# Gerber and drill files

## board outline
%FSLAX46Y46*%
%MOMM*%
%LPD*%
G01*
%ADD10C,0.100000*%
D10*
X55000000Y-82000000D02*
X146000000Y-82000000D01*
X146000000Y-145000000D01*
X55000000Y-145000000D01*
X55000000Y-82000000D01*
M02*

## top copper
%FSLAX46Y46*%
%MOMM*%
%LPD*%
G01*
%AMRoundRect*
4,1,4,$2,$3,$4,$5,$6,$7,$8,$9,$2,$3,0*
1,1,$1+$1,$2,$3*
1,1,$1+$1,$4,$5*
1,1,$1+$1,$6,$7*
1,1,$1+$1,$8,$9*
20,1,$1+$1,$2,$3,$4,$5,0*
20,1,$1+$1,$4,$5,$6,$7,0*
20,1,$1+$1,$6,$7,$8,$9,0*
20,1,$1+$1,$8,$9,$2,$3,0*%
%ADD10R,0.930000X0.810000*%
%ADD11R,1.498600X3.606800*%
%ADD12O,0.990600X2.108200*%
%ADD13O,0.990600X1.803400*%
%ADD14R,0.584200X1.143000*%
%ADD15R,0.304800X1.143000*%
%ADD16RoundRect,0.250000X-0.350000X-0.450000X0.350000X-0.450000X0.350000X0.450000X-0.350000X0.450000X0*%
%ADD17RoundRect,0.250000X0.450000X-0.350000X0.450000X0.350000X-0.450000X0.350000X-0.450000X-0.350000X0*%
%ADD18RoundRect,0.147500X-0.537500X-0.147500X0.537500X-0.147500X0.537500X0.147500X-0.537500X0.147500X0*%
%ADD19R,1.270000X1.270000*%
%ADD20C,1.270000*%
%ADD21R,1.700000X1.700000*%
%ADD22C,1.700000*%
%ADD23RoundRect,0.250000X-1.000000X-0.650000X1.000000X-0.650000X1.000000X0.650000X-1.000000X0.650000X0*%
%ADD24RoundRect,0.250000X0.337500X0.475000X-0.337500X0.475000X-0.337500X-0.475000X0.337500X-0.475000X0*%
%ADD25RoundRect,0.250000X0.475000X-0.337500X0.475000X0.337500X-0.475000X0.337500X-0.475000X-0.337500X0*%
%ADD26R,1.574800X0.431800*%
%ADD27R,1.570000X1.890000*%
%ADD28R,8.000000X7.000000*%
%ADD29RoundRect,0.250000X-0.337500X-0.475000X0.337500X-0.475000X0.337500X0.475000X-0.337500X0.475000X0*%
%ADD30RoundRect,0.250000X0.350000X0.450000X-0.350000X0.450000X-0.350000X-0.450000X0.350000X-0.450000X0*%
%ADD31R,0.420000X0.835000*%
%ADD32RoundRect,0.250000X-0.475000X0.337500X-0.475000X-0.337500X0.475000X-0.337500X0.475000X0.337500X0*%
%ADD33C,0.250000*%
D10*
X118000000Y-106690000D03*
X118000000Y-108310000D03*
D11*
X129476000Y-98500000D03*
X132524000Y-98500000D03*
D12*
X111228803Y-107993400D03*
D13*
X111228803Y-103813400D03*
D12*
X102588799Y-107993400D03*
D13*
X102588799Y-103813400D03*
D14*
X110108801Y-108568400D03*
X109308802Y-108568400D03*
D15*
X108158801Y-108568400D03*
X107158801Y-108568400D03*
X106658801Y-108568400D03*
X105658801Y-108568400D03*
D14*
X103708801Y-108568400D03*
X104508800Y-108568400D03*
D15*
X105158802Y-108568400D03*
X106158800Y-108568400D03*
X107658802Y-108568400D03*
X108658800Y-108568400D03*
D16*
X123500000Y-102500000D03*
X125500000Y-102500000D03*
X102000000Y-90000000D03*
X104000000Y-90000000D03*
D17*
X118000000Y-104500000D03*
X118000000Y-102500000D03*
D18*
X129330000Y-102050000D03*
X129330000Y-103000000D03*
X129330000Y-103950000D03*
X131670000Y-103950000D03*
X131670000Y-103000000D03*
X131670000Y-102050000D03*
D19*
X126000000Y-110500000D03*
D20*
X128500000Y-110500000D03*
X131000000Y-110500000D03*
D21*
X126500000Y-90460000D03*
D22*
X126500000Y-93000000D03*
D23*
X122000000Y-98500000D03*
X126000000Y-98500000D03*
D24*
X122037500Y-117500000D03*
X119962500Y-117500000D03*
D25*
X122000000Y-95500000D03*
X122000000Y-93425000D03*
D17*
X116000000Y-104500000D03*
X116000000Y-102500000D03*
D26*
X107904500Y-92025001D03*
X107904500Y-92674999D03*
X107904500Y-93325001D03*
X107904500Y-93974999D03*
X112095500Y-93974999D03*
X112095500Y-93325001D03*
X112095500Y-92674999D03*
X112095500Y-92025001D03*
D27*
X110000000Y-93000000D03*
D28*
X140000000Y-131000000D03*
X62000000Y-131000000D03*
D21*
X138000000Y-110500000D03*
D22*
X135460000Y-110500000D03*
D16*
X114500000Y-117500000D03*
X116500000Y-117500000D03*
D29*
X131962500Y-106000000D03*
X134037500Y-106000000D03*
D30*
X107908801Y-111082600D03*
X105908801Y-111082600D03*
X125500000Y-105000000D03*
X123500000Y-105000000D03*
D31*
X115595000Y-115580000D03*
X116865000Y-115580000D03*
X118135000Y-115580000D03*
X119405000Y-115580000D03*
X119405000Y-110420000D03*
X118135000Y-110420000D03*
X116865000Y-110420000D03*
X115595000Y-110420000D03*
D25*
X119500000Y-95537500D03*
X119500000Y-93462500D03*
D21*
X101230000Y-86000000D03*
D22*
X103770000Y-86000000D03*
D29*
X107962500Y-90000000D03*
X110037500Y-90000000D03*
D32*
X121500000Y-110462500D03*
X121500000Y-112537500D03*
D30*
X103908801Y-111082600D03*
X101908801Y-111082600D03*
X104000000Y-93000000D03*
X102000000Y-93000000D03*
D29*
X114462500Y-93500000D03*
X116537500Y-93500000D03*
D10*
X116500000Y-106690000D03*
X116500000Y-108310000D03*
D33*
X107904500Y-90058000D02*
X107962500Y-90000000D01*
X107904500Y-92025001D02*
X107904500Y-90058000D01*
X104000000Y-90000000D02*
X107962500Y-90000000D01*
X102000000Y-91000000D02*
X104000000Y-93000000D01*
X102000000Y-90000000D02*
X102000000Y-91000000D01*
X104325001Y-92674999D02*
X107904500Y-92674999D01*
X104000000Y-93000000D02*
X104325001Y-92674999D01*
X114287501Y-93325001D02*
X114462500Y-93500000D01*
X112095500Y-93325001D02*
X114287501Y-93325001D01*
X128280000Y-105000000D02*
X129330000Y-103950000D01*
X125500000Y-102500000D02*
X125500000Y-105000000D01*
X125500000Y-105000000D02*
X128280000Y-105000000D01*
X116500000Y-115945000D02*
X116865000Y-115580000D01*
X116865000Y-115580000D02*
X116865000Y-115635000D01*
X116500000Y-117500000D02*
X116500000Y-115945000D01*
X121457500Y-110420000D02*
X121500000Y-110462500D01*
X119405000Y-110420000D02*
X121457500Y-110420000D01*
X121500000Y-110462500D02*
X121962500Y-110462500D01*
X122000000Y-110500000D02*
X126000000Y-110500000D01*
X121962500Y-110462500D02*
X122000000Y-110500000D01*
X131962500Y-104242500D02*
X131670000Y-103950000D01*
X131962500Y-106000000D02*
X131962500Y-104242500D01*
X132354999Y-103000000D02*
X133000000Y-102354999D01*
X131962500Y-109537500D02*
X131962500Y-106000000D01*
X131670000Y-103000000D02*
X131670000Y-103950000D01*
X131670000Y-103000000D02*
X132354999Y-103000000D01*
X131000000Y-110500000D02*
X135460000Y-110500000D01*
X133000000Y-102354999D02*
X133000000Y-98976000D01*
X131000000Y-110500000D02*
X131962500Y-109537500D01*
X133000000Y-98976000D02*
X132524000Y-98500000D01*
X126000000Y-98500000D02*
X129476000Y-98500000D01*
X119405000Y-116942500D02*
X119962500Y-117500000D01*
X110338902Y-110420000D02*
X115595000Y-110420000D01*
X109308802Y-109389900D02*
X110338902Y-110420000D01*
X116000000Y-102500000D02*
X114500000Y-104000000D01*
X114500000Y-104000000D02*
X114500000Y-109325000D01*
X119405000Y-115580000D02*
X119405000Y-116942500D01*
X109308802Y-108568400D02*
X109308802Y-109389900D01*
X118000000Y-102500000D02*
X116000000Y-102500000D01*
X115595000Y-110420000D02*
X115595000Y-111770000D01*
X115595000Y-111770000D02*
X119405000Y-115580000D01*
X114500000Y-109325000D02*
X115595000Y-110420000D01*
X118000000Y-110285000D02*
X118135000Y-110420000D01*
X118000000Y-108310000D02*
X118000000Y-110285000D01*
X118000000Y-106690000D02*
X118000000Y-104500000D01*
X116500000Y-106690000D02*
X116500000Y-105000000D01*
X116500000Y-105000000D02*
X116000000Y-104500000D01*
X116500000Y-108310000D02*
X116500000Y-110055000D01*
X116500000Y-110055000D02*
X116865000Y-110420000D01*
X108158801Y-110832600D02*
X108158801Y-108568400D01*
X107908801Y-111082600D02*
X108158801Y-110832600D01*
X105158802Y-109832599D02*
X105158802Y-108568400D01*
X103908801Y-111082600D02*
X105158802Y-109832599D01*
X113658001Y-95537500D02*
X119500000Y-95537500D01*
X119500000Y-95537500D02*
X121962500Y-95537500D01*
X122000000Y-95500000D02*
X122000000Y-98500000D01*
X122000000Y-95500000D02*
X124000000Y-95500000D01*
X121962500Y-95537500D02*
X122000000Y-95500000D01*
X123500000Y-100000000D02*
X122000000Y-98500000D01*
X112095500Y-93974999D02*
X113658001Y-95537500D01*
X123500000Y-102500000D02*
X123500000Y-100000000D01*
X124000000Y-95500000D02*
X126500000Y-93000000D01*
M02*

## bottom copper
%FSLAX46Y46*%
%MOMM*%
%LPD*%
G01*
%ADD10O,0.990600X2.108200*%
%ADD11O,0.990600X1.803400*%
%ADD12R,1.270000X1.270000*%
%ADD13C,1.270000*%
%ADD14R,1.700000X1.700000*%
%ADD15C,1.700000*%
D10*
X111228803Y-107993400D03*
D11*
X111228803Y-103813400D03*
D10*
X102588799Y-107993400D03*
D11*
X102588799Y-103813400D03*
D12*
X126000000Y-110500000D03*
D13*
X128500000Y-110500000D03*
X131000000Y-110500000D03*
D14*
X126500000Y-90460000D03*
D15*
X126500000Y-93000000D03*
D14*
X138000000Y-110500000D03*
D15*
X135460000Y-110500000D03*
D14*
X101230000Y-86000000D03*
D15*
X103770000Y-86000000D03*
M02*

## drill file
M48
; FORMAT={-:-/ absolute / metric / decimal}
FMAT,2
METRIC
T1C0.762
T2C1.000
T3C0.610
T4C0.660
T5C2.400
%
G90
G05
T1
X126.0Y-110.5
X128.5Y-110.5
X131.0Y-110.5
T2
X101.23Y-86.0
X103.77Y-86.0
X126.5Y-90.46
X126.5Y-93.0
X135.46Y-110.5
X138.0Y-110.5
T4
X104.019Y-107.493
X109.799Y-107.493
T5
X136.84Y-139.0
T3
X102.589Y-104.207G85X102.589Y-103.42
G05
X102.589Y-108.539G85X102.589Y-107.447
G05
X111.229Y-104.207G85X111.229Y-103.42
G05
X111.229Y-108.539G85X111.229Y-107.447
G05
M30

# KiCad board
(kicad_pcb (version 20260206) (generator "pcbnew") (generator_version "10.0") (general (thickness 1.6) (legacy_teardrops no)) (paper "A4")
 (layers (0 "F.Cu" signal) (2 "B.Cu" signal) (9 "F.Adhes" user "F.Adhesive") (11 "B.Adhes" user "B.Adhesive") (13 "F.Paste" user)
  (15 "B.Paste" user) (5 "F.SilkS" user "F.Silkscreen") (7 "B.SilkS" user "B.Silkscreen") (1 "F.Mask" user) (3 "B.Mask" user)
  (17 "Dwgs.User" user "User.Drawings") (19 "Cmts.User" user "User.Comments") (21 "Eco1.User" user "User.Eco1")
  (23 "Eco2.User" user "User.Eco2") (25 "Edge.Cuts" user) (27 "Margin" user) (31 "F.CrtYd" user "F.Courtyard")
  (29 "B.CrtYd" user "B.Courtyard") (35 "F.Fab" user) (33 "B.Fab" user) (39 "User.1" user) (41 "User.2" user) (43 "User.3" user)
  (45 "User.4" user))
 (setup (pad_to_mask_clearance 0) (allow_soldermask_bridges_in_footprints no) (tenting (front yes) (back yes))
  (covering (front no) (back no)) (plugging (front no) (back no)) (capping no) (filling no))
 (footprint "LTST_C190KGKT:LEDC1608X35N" (layer "F.Cu") (at 118 107.5 90)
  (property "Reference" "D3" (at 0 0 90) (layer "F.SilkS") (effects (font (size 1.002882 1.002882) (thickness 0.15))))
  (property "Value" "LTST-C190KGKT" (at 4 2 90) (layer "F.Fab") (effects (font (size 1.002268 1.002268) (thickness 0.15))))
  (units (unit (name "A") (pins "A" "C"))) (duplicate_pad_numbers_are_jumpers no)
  (pad "A" smd rect (at 0.81 0 90) (size 0.81 0.93) (layers "F.Cu" "F.Mask" "F.Paste") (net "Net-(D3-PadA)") (solder_mask_margin 0.102))
  (pad "C" smd rect (at -0.81 0 90) (size 0.81 0.93) (layers "F.Cu" "F.Mask" "F.Paste") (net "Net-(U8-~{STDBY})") (solder_mask_margin 0.102)))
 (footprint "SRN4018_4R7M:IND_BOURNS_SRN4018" (layer "F.Cu") (at 131 98.5)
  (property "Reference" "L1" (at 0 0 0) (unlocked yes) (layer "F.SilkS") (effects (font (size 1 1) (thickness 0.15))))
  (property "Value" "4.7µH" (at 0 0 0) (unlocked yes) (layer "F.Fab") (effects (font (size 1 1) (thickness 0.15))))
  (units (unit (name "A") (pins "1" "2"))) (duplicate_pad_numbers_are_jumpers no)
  (pad "1" smd rect (at -1.524 0) (size 1.4986 3.6068) (layers "F.Cu" "F.Mask" "F.Paste") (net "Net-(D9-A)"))
  (pad "2" smd rect (at 1.524 0) (size 1.4986 3.6068) (layers "F.Cu" "F.Mask" "F.Paste") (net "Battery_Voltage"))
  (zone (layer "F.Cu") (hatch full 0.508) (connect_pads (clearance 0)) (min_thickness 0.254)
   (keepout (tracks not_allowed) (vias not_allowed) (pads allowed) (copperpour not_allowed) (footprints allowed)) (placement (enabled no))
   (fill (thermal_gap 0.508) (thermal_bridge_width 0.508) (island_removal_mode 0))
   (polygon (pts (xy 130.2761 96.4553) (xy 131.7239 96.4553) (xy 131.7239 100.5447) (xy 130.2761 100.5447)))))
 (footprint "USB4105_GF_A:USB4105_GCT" (layer "F.Cu") (at 106.908801 105.0826 180)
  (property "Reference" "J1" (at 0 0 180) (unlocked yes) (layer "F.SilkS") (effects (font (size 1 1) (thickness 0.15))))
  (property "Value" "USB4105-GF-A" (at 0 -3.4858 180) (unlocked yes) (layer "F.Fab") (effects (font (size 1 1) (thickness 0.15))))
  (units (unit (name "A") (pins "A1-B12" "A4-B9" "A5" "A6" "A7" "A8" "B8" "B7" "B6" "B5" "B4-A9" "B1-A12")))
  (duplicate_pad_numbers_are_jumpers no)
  (pad "" np_thru_hole oval (at -4.320002 -2.9108 180) (size 0.9906 2.1082) (drill oval 0.6096 1.7018) (layers "*.Cu" "*.Mask"))
  (pad "" np_thru_hole oval (at -4.320002 1.2692 180) (size 0.9906 1.8034) (drill oval 0.6096 1.397) (layers "*.Cu" "*.Mask"))
  (pad "" np_thru_hole circle (at -2.889999 -2.410801 180) (size 0.6604 0.6604) (drill 0.6604) (layers "*.Cu" "*.Mask"))
  (pad "" np_thru_hole circle (at 2.889999 -2.410801 180) (size 0.6604 0.6604) (drill 0.6604) (layers "*.Cu" "*.Mask"))
  (pad "" np_thru_hole oval (at 4.320002 -2.9108 180) (size 0.9906 2.1082) (drill oval 0.6096 1.7018) (layers "*.Cu" "*.Mask"))
  (pad "" np_thru_hole oval (at 4.320002 1.2692 180) (size 0.9906 1.8034) (drill oval 0.6096 1.397) (layers "*.Cu" "*.Mask"))
  (pad "A1-B12" smd rect (at -3.2 -3.4858 180) (size 0.5842 1.143) (layers "F.Cu" "F.Mask" "F.Paste") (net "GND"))
  (pad "A4-B9" smd rect (at -2.400001 -3.4858 180) (size 0.5842 1.143) (layers "F.Cu" "F.Mask" "F.Paste") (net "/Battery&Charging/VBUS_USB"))
  (pad "A5" smd rect (at -1.25 -3.4858 180) (size 0.3048 1.143) (layers "F.Cu" "F.Mask" "F.Paste") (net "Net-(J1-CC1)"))
  (pad "A6" smd rect (at -0.25 -3.4858 180) (size 0.3048 1.143) (layers "F.Cu" "F.Mask" "F.Paste") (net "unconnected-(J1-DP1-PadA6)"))
  (pad "A7" smd rect (at 0.25 -3.4858 180) (size 0.3048 1.143) (layers "F.Cu" "F.Mask" "F.Paste") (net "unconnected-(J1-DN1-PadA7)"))
  (pad "A8" smd rect (at 1.25 -3.4858 180) (size 0.3048 1.143) (layers "F.Cu" "F.Mask" "F.Paste") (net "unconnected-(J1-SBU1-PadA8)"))
  (pad "B1-A12" smd rect (at 3.2 -3.4858 180) (size 0.5842 1.143) (layers "F.Cu" "F.Mask" "F.Paste") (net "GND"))
  (pad "B4-A9" smd rect (at 2.400001 -3.4858 180) (size 0.5842 1.143) (layers "F.Cu" "F.Mask" "F.Paste")
   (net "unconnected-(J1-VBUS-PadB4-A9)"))
  (pad "B5" smd rect (at 1.749999 -3.4858 180) (size 0.3048 1.143) (layers "F.Cu" "F.Mask" "F.Paste") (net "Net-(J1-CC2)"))
  (pad "B6" smd rect (at 0.750001 -3.4858 180) (size 0.3048 1.143) (layers "F.Cu" "F.Mask" "F.Paste") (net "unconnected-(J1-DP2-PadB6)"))
  (pad "B7" smd rect (at -0.750001 -3.4858 180) (size 0.3048 1.143) (layers "F.Cu" "F.Mask" "F.Paste") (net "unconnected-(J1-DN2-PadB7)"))
  (pad "B8" smd rect (at -1.749999 -3.4858 180) (size 0.3048 1.143) (layers "F.Cu" "F.Mask" "F.Paste") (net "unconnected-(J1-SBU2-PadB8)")))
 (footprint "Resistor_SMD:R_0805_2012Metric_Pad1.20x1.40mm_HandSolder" (layer "F.Cu") (at 124.5 102.5)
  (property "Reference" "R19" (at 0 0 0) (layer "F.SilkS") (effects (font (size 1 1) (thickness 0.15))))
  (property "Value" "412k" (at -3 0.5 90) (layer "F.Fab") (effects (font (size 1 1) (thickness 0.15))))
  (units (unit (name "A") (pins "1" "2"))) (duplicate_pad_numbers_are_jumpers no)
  (pad "1" smd roundrect (at -1 0) (size 1.2 1.4) (layers "F.Cu" "F.Mask" "F.Paste") (roundrect_rratio 0.208333)
   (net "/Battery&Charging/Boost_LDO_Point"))
  (pad "2" smd roundrect (at 1 0) (size 1.2 1.4) (layers "F.Cu" "F.Mask" "F.Paste") (roundrect_rratio 0.208333) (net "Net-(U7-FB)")))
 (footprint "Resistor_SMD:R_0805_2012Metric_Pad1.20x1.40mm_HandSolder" (layer "F.Cu") (at 103 90)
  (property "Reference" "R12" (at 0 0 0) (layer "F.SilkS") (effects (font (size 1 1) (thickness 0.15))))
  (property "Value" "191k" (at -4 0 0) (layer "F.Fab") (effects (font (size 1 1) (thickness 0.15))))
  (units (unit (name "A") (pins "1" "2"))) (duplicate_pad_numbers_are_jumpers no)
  (pad "1" smd roundrect (at -1 0) (size 1.2 1.4) (layers "F.Cu" "F.Mask" "F.Paste") (roundrect_rratio 0.208333) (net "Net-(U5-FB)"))
  (pad "2" smd roundrect (at 1 0) (size 1.2 1.4) (layers "F.Cu" "F.Mask" "F.Paste") (roundrect_rratio 0.208333) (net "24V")))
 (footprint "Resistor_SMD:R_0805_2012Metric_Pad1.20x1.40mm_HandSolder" (layer "F.Cu") (at 118 103.5 90)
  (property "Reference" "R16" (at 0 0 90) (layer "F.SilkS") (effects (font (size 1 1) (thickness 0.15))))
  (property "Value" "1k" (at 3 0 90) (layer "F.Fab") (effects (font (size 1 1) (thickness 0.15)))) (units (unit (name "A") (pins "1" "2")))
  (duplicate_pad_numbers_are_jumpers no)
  (pad "1" smd roundrect (at -1 0 90) (size 1.2 1.4) (layers "F.Cu" "F.Mask" "F.Paste") (roundrect_rratio 0.208333) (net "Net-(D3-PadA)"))
  (pad "2" smd roundrect (at 1 0 90) (size 1.2 1.4) (layers "F.Cu" "F.Mask" "F.Paste") (roundrect_rratio 0.208333)
   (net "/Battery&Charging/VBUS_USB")))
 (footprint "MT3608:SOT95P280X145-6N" (layer "F.Cu") (at 130.5 103)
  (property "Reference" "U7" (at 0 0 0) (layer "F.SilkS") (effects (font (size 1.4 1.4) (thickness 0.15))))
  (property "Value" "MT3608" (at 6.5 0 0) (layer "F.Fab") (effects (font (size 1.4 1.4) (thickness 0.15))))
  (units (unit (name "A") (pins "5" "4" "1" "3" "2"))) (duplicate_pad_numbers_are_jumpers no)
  (pad "1" smd roundrect (at -1.17 -0.95) (size 1.37 0.59) (layers "F.Cu" "F.Mask" "F.Paste") (roundrect_rratio 0.25) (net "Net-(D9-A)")
   (solder_mask_margin 0.102))
  (pad "2" smd roundrect (at -1.17 0) (size 1.37 0.59) (layers "F.Cu" "F.Mask" "F.Paste") (roundrect_rratio 0.25) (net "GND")
   (solder_mask_margin 0.102))
  (pad "3" smd roundrect (at -1.17 0.95) (size 1.37 0.59) (layers "F.Cu" "F.Mask" "F.Paste") (roundrect_rratio 0.25) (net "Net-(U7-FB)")
   (solder_mask_margin 0.102))
  (pad "4" smd roundrect (at 1.17 0.95) (size 1.37 0.59) (layers "F.Cu" "F.Mask" "F.Paste") (roundrect_rratio 0.25) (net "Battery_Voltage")
   (solder_mask_margin 0.102))
  (pad "5" smd roundrect (at 1.17 0) (size 1.37 0.59) (layers "F.Cu" "F.Mask" "F.Paste") (roundrect_rratio 0.25) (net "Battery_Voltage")
   (solder_mask_margin 0.102))
  (pad "6" smd roundrect (at 1.17 -0.95) (size 1.37 0.59) (layers "F.Cu" "F.Mask" "F.Paste") (roundrect_rratio 0.25)
   (solder_mask_margin 0.102)))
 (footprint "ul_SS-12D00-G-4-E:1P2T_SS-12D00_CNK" (layer "F.Cu") (at 126 110.5 90)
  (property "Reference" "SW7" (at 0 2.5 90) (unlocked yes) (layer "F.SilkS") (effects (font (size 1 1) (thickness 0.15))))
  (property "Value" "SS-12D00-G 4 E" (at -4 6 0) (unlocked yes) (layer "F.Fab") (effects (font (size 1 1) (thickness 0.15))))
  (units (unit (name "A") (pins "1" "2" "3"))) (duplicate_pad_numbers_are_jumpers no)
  (pad "1" thru_hole rect (at 0 0 90) (size 1.27 1.27) (drill 0.762) (layers "*.Cu" "*.Mask") (remove_unused_layers no) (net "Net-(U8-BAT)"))
  (pad "2" thru_hole circle (at 0 2.5 90) (size 1.27 1.27) (drill 0.762) (layers "*.Cu" "*.Mask") (remove_unused_layers no)
   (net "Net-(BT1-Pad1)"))
  (pad "3" thru_hole circle (at 0 5 90) (size 1.27 1.27) (drill 0.762) (layers "*.Cu" "*.Mask") (remove_unused_layers no)
   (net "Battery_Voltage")))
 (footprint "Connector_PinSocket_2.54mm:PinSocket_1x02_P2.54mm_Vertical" (layer "F.Cu") (at 126.5 90.46)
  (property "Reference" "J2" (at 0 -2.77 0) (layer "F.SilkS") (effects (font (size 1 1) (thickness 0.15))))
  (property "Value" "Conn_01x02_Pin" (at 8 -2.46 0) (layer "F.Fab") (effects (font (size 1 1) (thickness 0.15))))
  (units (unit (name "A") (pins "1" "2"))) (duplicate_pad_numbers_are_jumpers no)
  (pad "1" thru_hole rect (at 0 0) (size 1.7 1.7) (drill 1) (layers "*.Cu" "*.Mask") (remove_unused_layers no) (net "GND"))
  (pad "2" thru_hole circle (at 0 2.54) (size 1.7 1.7) (drill 1) (layers "*.Cu" "*.Mask") (remove_unused_layers no)
   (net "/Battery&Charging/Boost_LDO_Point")))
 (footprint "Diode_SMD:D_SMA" (layer "F.Cu") (at 124 98.5)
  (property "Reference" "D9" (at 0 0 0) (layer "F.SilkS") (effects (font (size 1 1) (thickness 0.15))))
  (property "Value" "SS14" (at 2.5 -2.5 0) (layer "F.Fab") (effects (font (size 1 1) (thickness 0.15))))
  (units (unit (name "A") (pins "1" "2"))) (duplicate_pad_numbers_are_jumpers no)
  (pad "1" smd roundrect (at -2 0) (size 2.5 1.8) (layers "F.Cu" "F.Mask" "F.Paste") (roundrect_rratio 0.1388888889)
   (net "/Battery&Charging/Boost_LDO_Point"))
  (pad "2" smd roundrect (at 2 0) (size 2.5 1.8) (layers "F.Cu" "F.Mask" "F.Paste") (roundrect_rratio 0.1388888889) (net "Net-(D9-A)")))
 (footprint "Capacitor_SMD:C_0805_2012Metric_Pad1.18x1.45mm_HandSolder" (layer "F.Cu") (at 121 117.5 180)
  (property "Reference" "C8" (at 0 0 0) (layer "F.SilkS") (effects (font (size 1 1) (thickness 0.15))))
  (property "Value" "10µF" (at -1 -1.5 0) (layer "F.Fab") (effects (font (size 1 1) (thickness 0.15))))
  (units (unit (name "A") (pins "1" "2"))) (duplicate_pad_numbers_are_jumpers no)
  (pad "1" smd roundrect (at -1.0375 0 180) (size 1.175 1.45) (layers "F.Cu" "F.Mask" "F.Paste") (roundrect_rratio 0.212766) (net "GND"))
  (pad "2" smd roundrect (at 1.0375 0 180) (size 1.175 1.45) (layers "F.Cu" "F.Mask" "F.Paste") (roundrect_rratio 0.212766)
   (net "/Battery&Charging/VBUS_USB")))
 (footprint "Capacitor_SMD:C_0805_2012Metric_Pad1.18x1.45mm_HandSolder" (layer "F.Cu") (at 122 94.4625 90)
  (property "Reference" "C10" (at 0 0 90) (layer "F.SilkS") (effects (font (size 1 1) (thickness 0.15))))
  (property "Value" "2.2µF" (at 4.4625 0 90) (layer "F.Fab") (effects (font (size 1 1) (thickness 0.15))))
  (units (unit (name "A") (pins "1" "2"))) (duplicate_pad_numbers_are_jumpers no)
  (pad "1" smd roundrect (at -1.0375 0 90) (size 1.175 1.45) (layers "F.Cu" "F.Mask" "F.Paste") (roundrect_rratio 0.212766)
   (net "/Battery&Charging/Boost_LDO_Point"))
  (pad "2" smd roundrect (at 1.0375 0 90) (size 1.175 1.45) (layers "F.Cu" "F.Mask" "F.Paste") (roundrect_rratio 0.212766) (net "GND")))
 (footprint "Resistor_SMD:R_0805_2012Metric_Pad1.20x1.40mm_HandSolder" (layer "F.Cu") (at 116 103.5 90)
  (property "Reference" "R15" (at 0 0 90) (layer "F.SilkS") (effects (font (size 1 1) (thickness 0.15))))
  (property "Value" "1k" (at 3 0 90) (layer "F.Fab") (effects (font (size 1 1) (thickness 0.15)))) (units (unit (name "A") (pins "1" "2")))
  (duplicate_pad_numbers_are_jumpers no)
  (pad "1" smd roundrect (at -1 0 90) (size 1.2 1.4) (layers "F.Cu" "F.Mask" "F.Paste") (roundrect_rratio 0.208333) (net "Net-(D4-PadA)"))
  (pad "2" smd roundrect (at 1 0 90) (size 1.2 1.4) (layers "F.Cu" "F.Mask" "F.Paste") (roundrect_rratio 0.208333)
   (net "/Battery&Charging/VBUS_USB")))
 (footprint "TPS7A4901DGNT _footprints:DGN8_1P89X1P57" (layer "F.Cu") (at 110 93)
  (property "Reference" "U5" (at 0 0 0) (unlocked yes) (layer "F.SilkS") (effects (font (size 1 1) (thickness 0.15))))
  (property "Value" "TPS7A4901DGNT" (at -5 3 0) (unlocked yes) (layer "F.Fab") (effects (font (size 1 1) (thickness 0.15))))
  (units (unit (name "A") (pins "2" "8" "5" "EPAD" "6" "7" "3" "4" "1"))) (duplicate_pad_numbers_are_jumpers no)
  (pad "1" smd rect (at -2.0955 -0.974999) (size 1.5748 0.4318) (layers "F.Cu" "F.Mask" "F.Paste") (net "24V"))
  (pad "2" smd rect (at -2.0955 -0.325001) (size 1.5748 0.4318) (layers "F.Cu" "F.Mask" "F.Paste") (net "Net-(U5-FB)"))
  (pad "3" smd rect (at -2.0955 0.325001) (size 1.5748 0.4318) (layers "F.Cu" "F.Mask" "F.Paste") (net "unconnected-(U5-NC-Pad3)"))
  (pad "4" smd rect (at -2.0955 0.974999) (size 1.5748 0.4318) (layers "F.Cu" "F.Mask" "F.Paste") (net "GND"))
  (pad "5" smd rect (at 2.0955 0.974999) (size 1.5748 0.4318) (layers "F.Cu" "F.Mask" "F.Paste") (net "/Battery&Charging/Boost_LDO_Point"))
  (pad "6" smd rect (at 2.0955 0.325001) (size 1.5748 0.4318) (layers "F.Cu" "F.Mask" "F.Paste") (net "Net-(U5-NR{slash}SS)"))
  (pad "7" smd rect (at 2.0955 -0.325001) (size 1.5748 0.4318) (layers "F.Cu" "F.Mask" "F.Paste") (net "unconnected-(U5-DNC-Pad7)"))
  (pad "8" smd rect (at 2.0955 -0.974999) (size 1.5748 0.4318) (layers "F.Cu" "F.Mask" "F.Paste") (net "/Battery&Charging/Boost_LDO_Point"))
  (pad "EPAD" smd rect (at 0 0) (size 1.57 1.89) (layers "F.Cu" "F.Mask" "F.Paste") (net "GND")))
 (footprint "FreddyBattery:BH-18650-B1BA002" (layer "F.Cu") (at 101 131 180)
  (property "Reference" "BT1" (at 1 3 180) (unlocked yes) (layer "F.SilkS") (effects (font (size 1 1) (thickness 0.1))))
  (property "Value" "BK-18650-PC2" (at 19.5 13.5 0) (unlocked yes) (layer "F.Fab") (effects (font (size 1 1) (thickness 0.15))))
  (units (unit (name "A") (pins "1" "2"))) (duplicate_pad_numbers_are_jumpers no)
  (pad "" np_thru_hole circle (at -35.84 -8 180) (size 2.4 2.4) (drill 2.4) (layers "*.Cu" "*.Mask"))
  (pad "1" smd rect (at -39 0 180) (size 8 7) (layers "F.Cu" "F.Mask" "F.Paste") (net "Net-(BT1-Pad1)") (thermal_bridge_angle 45))
  (pad "2" smd rect (at 39 0 180) (size 8 7) (layers "F.Cu" "F.Mask" "F.Paste") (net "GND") (thermal_bridge_angle 45)))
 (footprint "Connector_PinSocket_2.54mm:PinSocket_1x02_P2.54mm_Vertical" (layer "F.Cu") (at 138 110.5 -90)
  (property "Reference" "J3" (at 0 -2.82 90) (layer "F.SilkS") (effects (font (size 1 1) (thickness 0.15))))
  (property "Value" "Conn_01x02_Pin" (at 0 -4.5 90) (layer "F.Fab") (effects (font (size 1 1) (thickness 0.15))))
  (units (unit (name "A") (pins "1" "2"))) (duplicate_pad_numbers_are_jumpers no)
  (pad "1" thru_hole rect (at 0 0 270) (size 1.7 1.7) (drill 1) (layers "*.Cu" "*.Mask") (remove_unused_layers no) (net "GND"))
  (pad "2" thru_hole circle (at 0 2.54 270) (size 1.7 1.7) (drill 1) (layers "*.Cu" "*.Mask") (remove_unused_layers no)
   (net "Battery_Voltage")))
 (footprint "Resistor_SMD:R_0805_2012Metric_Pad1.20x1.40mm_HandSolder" (layer "F.Cu") (at 115.5 117.5)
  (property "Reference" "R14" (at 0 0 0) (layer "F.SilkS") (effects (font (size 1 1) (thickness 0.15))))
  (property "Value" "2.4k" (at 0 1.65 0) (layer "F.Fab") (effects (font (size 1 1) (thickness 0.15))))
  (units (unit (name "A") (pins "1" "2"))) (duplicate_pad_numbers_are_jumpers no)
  (pad "1" smd roundrect (at -1 0) (size 1.2 1.4) (layers "F.Cu" "F.Mask" "F.Paste") (roundrect_rratio 0.208333) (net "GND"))
  (pad "2" smd roundrect (at 1 0) (size 1.2 1.4) (layers "F.Cu" "F.Mask" "F.Paste") (roundrect_rratio 0.208333) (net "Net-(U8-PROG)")))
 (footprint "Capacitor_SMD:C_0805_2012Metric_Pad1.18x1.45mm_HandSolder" (layer "F.Cu") (at 133 106)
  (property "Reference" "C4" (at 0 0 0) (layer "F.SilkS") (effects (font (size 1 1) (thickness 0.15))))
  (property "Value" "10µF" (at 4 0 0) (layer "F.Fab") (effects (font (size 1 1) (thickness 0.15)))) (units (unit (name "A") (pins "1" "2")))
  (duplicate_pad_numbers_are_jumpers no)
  (pad "1" smd roundrect (at -1.0375 0) (size 1.175 1.45) (layers "F.Cu" "F.Mask" "F.Paste") (roundrect_rratio 0.212766)
   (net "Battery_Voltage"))
  (pad "2" smd roundrect (at 1.0375 0) (size 1.175 1.45) (layers "F.Cu" "F.Mask" "F.Paste") (roundrect_rratio 0.212766) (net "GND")))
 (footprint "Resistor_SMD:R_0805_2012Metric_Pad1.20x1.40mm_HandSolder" (layer "F.Cu") (at 106.908801 111.0826 180)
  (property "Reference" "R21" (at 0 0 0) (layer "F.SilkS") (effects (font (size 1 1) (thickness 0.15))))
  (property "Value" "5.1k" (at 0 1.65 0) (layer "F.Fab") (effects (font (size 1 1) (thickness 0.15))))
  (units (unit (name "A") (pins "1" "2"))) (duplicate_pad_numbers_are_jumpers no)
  (pad "1" smd roundrect (at -1 0 180) (size 1.2 1.4) (layers "F.Cu" "F.Mask" "F.Paste") (roundrect_rratio 0.208333) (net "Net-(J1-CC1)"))
  (pad "2" smd roundrect (at 1 0 180) (size 1.2 1.4) (layers "F.Cu" "F.Mask" "F.Paste") (roundrect_rratio 0.208333) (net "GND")))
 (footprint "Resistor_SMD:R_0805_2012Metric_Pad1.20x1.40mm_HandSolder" (layer "F.Cu") (at 124.5 105 180)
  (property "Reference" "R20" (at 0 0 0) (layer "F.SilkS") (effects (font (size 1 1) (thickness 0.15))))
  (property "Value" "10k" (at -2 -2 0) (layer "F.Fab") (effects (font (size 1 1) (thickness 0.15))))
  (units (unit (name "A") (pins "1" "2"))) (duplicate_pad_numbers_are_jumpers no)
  (pad "1" smd roundrect (at -1 0 180) (size 1.2 1.4) (layers "F.Cu" "F.Mask" "F.Paste") (roundrect_rratio 0.208333) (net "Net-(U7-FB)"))
  (pad "2" smd roundrect (at 1 0 180) (size 1.2 1.4) (layers "F.Cu" "F.Mask" "F.Paste") (roundrect_rratio 0.208333) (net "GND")))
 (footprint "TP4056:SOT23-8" (layer "F.Cu") (at 117.5 113)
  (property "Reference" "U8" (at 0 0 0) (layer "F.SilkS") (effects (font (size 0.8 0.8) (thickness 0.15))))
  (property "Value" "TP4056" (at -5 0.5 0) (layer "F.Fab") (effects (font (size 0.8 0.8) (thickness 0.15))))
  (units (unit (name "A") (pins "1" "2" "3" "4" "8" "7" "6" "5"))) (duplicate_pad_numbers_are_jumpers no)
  (pad "1" smd rect (at -1.905 2.58) (size 0.42 0.835) (layers "F.Cu" "F.Mask" "F.Paste") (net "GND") (solder_mask_margin 0.102))
  (pad "2" smd rect (at -0.635 2.58) (size 0.42 0.835) (layers "F.Cu" "F.Mask" "F.Paste") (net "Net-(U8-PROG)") (solder_mask_margin 0.102))
  (pad "3" smd rect (at 0.635 2.58) (size 0.42 0.835) (layers "F.Cu" "F.Mask" "F.Paste") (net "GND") (solder_mask_margin 0.102))
  (pad "4" smd rect (at 1.905 2.58) (size 0.42 0.835) (layers "F.Cu" "F.Mask" "F.Paste") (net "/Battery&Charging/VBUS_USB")
   (solder_mask_margin 0.102))
  (pad "5" smd rect (at 1.905 -2.58) (size 0.42 0.835) (layers "F.Cu" "F.Mask" "F.Paste") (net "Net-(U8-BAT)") (solder_mask_margin 0.102))
  (pad "6" smd rect (at 0.635 -2.58) (size 0.42 0.835) (layers "F.Cu" "F.Mask" "F.Paste") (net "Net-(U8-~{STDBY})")
   (solder_mask_margin 0.102))
  (pad "7" smd rect (at -0.635 -2.58) (size 0.42 0.835) (layers "F.Cu" "F.Mask" "F.Paste") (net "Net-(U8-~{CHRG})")
   (solder_mask_margin 0.102))
  (pad "8" smd rect (at -1.905 -2.58) (size 0.42 0.835) (layers "F.Cu" "F.Mask" "F.Paste") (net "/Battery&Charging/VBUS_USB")
   (solder_mask_margin 0.102)))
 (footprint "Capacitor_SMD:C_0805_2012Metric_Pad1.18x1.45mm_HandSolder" (layer "F.Cu") (at 119.5 94.5 90)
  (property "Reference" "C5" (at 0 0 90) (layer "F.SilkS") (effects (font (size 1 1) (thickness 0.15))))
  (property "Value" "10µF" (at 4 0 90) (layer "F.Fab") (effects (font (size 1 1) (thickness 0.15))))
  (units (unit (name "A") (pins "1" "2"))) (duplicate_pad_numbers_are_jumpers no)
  (pad "1" smd roundrect (at -1.0375 0 90) (size 1.175 1.45) (layers "F.Cu" "F.Mask" "F.Paste") (roundrect_rratio 0.212766)
   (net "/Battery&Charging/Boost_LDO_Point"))
  (pad "2" smd roundrect (at 1.0375 0 90) (size 1.175 1.45) (layers "F.Cu" "F.Mask" "F.Paste") (roundrect_rratio 0.212766) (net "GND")))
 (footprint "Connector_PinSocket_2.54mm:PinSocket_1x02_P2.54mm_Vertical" (layer "F.Cu") (at 101.23 86 90)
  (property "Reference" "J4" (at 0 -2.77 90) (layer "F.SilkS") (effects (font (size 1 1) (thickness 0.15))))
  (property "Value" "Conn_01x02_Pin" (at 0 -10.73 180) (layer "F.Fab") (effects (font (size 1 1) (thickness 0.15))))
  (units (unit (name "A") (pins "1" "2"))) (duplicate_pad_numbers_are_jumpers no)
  (pad "1" thru_hole rect (at 0 0 90) (size 1.7 1.7) (drill 1) (layers "*.Cu" "*.Mask") (remove_unused_layers no) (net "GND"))
  (pad "2" thru_hole circle (at 0 2.54 90) (size 1.7 1.7) (drill 1) (layers "*.Cu" "*.Mask") (remove_unused_layers no) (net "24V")))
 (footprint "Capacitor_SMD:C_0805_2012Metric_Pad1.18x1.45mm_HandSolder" (layer "F.Cu") (at 109 90)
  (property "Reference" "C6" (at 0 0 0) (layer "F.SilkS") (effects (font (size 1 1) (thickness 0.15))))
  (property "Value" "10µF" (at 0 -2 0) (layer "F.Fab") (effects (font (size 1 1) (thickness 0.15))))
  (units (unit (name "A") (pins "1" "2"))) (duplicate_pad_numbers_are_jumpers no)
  (pad "1" smd roundrect (at -1.0375 0) (size 1.175 1.45) (layers "F.Cu" "F.Mask" "F.Paste") (roundrect_rratio 0.212766) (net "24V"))
  (pad "2" smd roundrect (at 1.0375 0) (size 1.175 1.45) (layers "F.Cu" "F.Mask" "F.Paste") (roundrect_rratio 0.212766) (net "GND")))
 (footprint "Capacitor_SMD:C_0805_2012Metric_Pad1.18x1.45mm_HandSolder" (layer "F.Cu") (at 121.5 111.5 -90)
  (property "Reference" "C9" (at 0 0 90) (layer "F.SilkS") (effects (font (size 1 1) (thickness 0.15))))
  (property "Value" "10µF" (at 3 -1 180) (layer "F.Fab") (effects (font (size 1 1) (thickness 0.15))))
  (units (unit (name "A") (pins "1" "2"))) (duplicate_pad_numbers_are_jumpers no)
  (pad "1" smd roundrect (at -1.0375 0 270) (size 1.175 1.45) (layers "F.Cu" "F.Mask" "F.Paste") (roundrect_rratio 0.212766)
   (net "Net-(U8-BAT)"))
  (pad "2" smd roundrect (at 1.0375 0 270) (size 1.175 1.45) (layers "F.Cu" "F.Mask" "F.Paste") (roundrect_rratio 0.212766) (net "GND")))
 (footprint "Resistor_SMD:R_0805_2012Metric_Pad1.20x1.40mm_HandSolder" (layer "F.Cu") (at 102.908801 111.0826 180)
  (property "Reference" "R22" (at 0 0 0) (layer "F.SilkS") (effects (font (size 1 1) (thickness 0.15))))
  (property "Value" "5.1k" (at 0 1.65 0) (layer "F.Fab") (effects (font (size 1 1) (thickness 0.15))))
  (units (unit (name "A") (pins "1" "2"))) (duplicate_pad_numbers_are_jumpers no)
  (pad "1" smd roundrect (at -1 0 180) (size 1.2 1.4) (layers "F.Cu" "F.Mask" "F.Paste") (roundrect_rratio 0.208333) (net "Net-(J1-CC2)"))
  (pad "2" smd roundrect (at 1 0 180) (size 1.2 1.4) (layers "F.Cu" "F.Mask" "F.Paste") (roundrect_rratio 0.208333) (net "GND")))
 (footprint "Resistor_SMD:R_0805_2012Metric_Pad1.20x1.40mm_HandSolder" (layer "F.Cu") (at 103 93 180)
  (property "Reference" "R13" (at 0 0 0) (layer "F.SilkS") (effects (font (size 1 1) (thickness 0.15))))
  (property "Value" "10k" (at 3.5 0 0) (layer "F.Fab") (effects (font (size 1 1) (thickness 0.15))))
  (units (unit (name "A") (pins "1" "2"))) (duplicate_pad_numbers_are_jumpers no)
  (pad "1" smd roundrect (at -1 0 180) (size 1.2 1.4) (layers "F.Cu" "F.Mask" "F.Paste") (roundrect_rratio 0.208333) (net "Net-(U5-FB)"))
  (pad "2" smd roundrect (at 1 0 180) (size 1.2 1.4) (layers "F.Cu" "F.Mask" "F.Paste") (roundrect_rratio 0.208333) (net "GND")))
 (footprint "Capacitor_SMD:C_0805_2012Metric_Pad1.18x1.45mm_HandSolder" (layer "F.Cu") (at 115.5 93.5)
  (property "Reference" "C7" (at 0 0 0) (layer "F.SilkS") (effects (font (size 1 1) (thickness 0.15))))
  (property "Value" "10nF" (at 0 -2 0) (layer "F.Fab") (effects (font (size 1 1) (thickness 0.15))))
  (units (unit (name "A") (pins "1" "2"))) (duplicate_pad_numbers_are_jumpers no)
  (pad "1" smd roundrect (at -1.0375 0) (size 1.175 1.45) (layers "F.Cu" "F.Mask" "F.Paste") (roundrect_rratio 0.212766)
   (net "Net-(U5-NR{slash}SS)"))
  (pad "2" smd roundrect (at 1.0375 0) (size 1.175 1.45) (layers "F.Cu" "F.Mask" "F.Paste") (roundrect_rratio 0.212766) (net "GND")))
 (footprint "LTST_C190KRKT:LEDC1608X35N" (layer "F.Cu") (at 116.5 107.5 90)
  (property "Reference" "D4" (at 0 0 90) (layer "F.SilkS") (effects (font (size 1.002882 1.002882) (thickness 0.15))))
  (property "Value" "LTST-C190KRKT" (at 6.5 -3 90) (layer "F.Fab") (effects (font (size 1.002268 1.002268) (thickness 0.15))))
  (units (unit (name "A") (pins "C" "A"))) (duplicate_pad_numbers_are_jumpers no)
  (pad "A" smd rect (at 0.81 0 90) (size 0.81 0.93) (layers "F.Cu" "F.Mask" "F.Paste") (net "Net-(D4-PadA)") (solder_mask_margin 0.102))
  (pad "C" smd rect (at -0.81 0 90) (size 0.81 0.93) (layers "F.Cu" "F.Mask" "F.Paste") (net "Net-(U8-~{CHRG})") (solder_mask_margin 0.102)))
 (gr_rect (start 55 82) (end 146 145) (stroke (width 0.1) (type solid)) (fill no) (layer "Edge.Cuts"))
 (segment (start 107.9045 90.058) (end 107.9625 90) (width 0.25) (layer "F.Cu") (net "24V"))
 (segment (start 107.9045 92.025001) (end 107.9045 90.058) (width 0.25) (layer "F.Cu") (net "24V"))
 (segment (start 104 90) (end 107.9625 90) (width 0.25) (layer "F.Cu") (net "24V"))
 (segment (start 102 91) (end 104 93) (width 0.25) (layer "F.Cu") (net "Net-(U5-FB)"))
 (segment (start 102 90) (end 102 91) (width 0.25) (layer "F.Cu") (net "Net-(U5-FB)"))
 (segment (start 104.325001 92.674999) (end 107.9045 92.674999) (width 0.25) (layer "F.Cu") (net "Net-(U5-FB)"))
 (segment (start 104 93) (end 104.325001 92.674999) (width 0.25) (layer "F.Cu") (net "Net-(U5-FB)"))
 (segment (start 114.287501 93.325001) (end 114.4625 93.5) (width 0.25) (layer "F.Cu") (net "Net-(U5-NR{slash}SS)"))
 (segment (start 112.0955 93.325001) (end 114.287501 93.325001) (width 0.25) (layer "F.Cu") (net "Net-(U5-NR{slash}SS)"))
 (segment (start 128.28 105) (end 129.33 103.95) (width 0.25) (layer "F.Cu") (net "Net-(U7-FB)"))
 (segment (start 125.5 102.5) (end 125.5 105) (width 0.25) (layer "F.Cu") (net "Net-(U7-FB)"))
 (segment (start 125.5 105) (end 128.28 105) (width 0.25) (layer "F.Cu") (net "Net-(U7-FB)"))
 (segment (start 116.5 115.945) (end 116.865 115.58) (width 0.25) (layer "F.Cu") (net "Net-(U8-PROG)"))
 (segment (start 116.865 115.58) (end 116.865 115.635) (width 0.25) (layer "F.Cu") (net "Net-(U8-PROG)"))
 (segment (start 116.5 117.5) (end 116.5 115.945) (width 0.25) (layer "F.Cu") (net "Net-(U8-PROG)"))
 (segment (start 121.4575 110.42) (end 121.5 110.4625) (width 0.25) (layer "F.Cu") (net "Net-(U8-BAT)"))
 (segment (start 119.405 110.42) (end 121.4575 110.42) (width 0.25) (layer "F.Cu") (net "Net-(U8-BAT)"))
 (segment (start 121.5 110.4625) (end 121.9625 110.4625) (width 0.25) (layer "F.Cu") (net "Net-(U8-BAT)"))
 (segment (start 122 110.5) (end 126 110.5) (width 0.25) (layer "F.Cu") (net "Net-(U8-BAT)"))
 (segment (start 121.9625 110.4625) (end 122 110.5) (width 0.25) (layer "F.Cu") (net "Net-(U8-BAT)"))
 (segment (start 131.9625 104.2425) (end 131.67 103.95) (width 0.25) (layer "F.Cu") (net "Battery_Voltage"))
 (segment (start 131.9625 106) (end 131.9625 104.2425) (width 0.25) (layer "F.Cu") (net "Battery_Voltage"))
 (segment (start 132.354999 103) (end 133 102.354999) (width 0.25) (layer "F.Cu") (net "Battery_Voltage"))
 (segment (start 131.9625 109.5375) (end 131.9625 106) (width 0.25) (layer "F.Cu") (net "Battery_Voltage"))
 (segment (start 131.67 103) (end 131.67 103.95) (width 0.25) (layer "F.Cu") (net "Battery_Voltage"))
 (segment (start 131.67 103) (end 132.354999 103) (width 0.25) (layer "F.Cu") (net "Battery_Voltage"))
 (segment (start 131 110.5) (end 135.46 110.5) (width 0.25) (layer "F.Cu") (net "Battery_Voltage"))
 (segment (start 133 102.354999) (end 133 98.976) (width 0.25) (layer "F.Cu") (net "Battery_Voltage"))
 (segment (start 131 110.5) (end 131.9625 109.5375) (width 0.25) (layer "F.Cu") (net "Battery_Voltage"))
 (segment (start 133 98.976) (end 132.524 98.5) (width 0.25) (layer "F.Cu") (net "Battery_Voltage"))
 (segment (start 126 98.5) (end 129.476 98.5) (width 0.25) (layer "F.Cu") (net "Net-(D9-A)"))
 (segment (start 119.405 116.9425) (end 119.9625 117.5) (width 0.25) (layer "F.Cu") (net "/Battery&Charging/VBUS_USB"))
 (segment (start 110.338902 110.42) (end 115.595 110.42) (width 0.25) (layer "F.Cu") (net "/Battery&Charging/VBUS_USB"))
 (segment (start 109.308802 109.3899) (end 110.338902 110.42) (width 0.25) (layer "F.Cu") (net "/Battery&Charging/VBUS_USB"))
 (segment (start 116 102.5) (end 114.5 104) (width 0.25) (layer "F.Cu") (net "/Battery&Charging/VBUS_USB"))
 (segment (start 114.5 104) (end 114.5 109.325) (width 0.25) (layer "F.Cu") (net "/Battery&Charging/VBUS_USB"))
 (segment (start 119.405 115.58) (end 119.405 116.9425) (width 0.25) (layer "F.Cu") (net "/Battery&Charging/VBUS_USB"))
 (segment (start 109.308802 108.5684) (end 109.308802 109.3899) (width 0.25) (layer "F.Cu") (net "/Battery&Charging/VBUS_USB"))
 (segment (start 118 102.5) (end 116 102.5) (width 0.25) (layer "F.Cu") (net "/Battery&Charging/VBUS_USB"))
 (segment (start 115.595 110.42) (end 115.595 111.77) (width 0.25) (layer "F.Cu") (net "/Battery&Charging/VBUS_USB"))
 (segment (start 115.595 111.77) (end 119.405 115.58) (width 0.25) (layer "F.Cu") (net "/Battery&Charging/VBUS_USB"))
 (segment (start 114.5 109.325) (end 115.595 110.42) (width 0.25) (layer "F.Cu") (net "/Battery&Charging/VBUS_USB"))
 (segment (start 118 110.285) (end 118.135 110.42) (width 0.25) (layer "F.Cu") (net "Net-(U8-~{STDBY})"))
 (segment (start 118 108.31) (end 118 110.285) (width 0.25) (layer "F.Cu") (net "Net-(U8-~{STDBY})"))
 (segment (start 118 106.69) (end 118 104.5) (width 0.25) (layer "F.Cu") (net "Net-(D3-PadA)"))
 (segment (start 116.5 106.69) (end 116.5 105) (width 0.25) (layer "F.Cu") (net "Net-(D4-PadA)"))
 (segment (start 116.5 105) (end 116 104.5) (width 0.25) (layer "F.Cu") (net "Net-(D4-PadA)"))
 (segment (start 116.5 108.31) (end 116.5 110.055) (width 0.25) (layer "F.Cu") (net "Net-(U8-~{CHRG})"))
 (segment (start 116.5 110.055) (end 116.865 110.42) (width 0.25) (layer "F.Cu") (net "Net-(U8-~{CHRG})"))
 (segment (start 108.158801 110.8326) (end 108.158801 108.5684) (width 0.25) (layer "F.Cu") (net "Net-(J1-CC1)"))
 (segment (start 107.908801 111.0826) (end 108.158801 110.8326) (width 0.25) (layer "F.Cu") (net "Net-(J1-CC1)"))
 (segment (start 105.158802 109.832599) (end 105.158802 108.5684) (width 0.25) (layer "F.Cu") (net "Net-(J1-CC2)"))
 (segment (start 103.908801 111.0826) (end 105.158802 109.832599) (width 0.25) (layer "F.Cu") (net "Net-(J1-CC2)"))
 (segment (start 113.658001 95.5375) (end 119.5 95.5375) (width 0.25) (layer "F.Cu") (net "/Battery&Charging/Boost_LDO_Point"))
 (segment (start 119.5 95.5375) (end 121.9625 95.5375) (width 0.25) (layer "F.Cu") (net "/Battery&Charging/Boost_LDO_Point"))
 (segment (start 122 95.5) (end 122 98.5) (width 0.25) (layer "F.Cu") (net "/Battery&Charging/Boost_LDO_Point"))
 (segment (start 122 95.5) (end 124 95.5) (width 0.25) (layer "F.Cu") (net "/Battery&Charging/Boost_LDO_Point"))
 (segment (start 121.9625 95.5375) (end 122 95.5) (width 0.25) (layer "F.Cu") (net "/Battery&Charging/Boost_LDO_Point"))
 (segment (start 123.5 100) (end 122 98.5) (width 0.25) (layer "F.Cu") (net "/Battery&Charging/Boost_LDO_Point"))
 (segment (start 112.0955 93.974999) (end 113.658001 95.5375) (width 0.25) (layer "F.Cu") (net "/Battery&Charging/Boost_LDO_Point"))
 (segment (start 123.5 102.5) (end 123.5 100) (width 0.25) (layer "F.Cu") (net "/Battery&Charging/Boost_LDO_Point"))
 (segment (start 124 95.5) (end 126.5 93) (width 0.25) (layer "F.Cu") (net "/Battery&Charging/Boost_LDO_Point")))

